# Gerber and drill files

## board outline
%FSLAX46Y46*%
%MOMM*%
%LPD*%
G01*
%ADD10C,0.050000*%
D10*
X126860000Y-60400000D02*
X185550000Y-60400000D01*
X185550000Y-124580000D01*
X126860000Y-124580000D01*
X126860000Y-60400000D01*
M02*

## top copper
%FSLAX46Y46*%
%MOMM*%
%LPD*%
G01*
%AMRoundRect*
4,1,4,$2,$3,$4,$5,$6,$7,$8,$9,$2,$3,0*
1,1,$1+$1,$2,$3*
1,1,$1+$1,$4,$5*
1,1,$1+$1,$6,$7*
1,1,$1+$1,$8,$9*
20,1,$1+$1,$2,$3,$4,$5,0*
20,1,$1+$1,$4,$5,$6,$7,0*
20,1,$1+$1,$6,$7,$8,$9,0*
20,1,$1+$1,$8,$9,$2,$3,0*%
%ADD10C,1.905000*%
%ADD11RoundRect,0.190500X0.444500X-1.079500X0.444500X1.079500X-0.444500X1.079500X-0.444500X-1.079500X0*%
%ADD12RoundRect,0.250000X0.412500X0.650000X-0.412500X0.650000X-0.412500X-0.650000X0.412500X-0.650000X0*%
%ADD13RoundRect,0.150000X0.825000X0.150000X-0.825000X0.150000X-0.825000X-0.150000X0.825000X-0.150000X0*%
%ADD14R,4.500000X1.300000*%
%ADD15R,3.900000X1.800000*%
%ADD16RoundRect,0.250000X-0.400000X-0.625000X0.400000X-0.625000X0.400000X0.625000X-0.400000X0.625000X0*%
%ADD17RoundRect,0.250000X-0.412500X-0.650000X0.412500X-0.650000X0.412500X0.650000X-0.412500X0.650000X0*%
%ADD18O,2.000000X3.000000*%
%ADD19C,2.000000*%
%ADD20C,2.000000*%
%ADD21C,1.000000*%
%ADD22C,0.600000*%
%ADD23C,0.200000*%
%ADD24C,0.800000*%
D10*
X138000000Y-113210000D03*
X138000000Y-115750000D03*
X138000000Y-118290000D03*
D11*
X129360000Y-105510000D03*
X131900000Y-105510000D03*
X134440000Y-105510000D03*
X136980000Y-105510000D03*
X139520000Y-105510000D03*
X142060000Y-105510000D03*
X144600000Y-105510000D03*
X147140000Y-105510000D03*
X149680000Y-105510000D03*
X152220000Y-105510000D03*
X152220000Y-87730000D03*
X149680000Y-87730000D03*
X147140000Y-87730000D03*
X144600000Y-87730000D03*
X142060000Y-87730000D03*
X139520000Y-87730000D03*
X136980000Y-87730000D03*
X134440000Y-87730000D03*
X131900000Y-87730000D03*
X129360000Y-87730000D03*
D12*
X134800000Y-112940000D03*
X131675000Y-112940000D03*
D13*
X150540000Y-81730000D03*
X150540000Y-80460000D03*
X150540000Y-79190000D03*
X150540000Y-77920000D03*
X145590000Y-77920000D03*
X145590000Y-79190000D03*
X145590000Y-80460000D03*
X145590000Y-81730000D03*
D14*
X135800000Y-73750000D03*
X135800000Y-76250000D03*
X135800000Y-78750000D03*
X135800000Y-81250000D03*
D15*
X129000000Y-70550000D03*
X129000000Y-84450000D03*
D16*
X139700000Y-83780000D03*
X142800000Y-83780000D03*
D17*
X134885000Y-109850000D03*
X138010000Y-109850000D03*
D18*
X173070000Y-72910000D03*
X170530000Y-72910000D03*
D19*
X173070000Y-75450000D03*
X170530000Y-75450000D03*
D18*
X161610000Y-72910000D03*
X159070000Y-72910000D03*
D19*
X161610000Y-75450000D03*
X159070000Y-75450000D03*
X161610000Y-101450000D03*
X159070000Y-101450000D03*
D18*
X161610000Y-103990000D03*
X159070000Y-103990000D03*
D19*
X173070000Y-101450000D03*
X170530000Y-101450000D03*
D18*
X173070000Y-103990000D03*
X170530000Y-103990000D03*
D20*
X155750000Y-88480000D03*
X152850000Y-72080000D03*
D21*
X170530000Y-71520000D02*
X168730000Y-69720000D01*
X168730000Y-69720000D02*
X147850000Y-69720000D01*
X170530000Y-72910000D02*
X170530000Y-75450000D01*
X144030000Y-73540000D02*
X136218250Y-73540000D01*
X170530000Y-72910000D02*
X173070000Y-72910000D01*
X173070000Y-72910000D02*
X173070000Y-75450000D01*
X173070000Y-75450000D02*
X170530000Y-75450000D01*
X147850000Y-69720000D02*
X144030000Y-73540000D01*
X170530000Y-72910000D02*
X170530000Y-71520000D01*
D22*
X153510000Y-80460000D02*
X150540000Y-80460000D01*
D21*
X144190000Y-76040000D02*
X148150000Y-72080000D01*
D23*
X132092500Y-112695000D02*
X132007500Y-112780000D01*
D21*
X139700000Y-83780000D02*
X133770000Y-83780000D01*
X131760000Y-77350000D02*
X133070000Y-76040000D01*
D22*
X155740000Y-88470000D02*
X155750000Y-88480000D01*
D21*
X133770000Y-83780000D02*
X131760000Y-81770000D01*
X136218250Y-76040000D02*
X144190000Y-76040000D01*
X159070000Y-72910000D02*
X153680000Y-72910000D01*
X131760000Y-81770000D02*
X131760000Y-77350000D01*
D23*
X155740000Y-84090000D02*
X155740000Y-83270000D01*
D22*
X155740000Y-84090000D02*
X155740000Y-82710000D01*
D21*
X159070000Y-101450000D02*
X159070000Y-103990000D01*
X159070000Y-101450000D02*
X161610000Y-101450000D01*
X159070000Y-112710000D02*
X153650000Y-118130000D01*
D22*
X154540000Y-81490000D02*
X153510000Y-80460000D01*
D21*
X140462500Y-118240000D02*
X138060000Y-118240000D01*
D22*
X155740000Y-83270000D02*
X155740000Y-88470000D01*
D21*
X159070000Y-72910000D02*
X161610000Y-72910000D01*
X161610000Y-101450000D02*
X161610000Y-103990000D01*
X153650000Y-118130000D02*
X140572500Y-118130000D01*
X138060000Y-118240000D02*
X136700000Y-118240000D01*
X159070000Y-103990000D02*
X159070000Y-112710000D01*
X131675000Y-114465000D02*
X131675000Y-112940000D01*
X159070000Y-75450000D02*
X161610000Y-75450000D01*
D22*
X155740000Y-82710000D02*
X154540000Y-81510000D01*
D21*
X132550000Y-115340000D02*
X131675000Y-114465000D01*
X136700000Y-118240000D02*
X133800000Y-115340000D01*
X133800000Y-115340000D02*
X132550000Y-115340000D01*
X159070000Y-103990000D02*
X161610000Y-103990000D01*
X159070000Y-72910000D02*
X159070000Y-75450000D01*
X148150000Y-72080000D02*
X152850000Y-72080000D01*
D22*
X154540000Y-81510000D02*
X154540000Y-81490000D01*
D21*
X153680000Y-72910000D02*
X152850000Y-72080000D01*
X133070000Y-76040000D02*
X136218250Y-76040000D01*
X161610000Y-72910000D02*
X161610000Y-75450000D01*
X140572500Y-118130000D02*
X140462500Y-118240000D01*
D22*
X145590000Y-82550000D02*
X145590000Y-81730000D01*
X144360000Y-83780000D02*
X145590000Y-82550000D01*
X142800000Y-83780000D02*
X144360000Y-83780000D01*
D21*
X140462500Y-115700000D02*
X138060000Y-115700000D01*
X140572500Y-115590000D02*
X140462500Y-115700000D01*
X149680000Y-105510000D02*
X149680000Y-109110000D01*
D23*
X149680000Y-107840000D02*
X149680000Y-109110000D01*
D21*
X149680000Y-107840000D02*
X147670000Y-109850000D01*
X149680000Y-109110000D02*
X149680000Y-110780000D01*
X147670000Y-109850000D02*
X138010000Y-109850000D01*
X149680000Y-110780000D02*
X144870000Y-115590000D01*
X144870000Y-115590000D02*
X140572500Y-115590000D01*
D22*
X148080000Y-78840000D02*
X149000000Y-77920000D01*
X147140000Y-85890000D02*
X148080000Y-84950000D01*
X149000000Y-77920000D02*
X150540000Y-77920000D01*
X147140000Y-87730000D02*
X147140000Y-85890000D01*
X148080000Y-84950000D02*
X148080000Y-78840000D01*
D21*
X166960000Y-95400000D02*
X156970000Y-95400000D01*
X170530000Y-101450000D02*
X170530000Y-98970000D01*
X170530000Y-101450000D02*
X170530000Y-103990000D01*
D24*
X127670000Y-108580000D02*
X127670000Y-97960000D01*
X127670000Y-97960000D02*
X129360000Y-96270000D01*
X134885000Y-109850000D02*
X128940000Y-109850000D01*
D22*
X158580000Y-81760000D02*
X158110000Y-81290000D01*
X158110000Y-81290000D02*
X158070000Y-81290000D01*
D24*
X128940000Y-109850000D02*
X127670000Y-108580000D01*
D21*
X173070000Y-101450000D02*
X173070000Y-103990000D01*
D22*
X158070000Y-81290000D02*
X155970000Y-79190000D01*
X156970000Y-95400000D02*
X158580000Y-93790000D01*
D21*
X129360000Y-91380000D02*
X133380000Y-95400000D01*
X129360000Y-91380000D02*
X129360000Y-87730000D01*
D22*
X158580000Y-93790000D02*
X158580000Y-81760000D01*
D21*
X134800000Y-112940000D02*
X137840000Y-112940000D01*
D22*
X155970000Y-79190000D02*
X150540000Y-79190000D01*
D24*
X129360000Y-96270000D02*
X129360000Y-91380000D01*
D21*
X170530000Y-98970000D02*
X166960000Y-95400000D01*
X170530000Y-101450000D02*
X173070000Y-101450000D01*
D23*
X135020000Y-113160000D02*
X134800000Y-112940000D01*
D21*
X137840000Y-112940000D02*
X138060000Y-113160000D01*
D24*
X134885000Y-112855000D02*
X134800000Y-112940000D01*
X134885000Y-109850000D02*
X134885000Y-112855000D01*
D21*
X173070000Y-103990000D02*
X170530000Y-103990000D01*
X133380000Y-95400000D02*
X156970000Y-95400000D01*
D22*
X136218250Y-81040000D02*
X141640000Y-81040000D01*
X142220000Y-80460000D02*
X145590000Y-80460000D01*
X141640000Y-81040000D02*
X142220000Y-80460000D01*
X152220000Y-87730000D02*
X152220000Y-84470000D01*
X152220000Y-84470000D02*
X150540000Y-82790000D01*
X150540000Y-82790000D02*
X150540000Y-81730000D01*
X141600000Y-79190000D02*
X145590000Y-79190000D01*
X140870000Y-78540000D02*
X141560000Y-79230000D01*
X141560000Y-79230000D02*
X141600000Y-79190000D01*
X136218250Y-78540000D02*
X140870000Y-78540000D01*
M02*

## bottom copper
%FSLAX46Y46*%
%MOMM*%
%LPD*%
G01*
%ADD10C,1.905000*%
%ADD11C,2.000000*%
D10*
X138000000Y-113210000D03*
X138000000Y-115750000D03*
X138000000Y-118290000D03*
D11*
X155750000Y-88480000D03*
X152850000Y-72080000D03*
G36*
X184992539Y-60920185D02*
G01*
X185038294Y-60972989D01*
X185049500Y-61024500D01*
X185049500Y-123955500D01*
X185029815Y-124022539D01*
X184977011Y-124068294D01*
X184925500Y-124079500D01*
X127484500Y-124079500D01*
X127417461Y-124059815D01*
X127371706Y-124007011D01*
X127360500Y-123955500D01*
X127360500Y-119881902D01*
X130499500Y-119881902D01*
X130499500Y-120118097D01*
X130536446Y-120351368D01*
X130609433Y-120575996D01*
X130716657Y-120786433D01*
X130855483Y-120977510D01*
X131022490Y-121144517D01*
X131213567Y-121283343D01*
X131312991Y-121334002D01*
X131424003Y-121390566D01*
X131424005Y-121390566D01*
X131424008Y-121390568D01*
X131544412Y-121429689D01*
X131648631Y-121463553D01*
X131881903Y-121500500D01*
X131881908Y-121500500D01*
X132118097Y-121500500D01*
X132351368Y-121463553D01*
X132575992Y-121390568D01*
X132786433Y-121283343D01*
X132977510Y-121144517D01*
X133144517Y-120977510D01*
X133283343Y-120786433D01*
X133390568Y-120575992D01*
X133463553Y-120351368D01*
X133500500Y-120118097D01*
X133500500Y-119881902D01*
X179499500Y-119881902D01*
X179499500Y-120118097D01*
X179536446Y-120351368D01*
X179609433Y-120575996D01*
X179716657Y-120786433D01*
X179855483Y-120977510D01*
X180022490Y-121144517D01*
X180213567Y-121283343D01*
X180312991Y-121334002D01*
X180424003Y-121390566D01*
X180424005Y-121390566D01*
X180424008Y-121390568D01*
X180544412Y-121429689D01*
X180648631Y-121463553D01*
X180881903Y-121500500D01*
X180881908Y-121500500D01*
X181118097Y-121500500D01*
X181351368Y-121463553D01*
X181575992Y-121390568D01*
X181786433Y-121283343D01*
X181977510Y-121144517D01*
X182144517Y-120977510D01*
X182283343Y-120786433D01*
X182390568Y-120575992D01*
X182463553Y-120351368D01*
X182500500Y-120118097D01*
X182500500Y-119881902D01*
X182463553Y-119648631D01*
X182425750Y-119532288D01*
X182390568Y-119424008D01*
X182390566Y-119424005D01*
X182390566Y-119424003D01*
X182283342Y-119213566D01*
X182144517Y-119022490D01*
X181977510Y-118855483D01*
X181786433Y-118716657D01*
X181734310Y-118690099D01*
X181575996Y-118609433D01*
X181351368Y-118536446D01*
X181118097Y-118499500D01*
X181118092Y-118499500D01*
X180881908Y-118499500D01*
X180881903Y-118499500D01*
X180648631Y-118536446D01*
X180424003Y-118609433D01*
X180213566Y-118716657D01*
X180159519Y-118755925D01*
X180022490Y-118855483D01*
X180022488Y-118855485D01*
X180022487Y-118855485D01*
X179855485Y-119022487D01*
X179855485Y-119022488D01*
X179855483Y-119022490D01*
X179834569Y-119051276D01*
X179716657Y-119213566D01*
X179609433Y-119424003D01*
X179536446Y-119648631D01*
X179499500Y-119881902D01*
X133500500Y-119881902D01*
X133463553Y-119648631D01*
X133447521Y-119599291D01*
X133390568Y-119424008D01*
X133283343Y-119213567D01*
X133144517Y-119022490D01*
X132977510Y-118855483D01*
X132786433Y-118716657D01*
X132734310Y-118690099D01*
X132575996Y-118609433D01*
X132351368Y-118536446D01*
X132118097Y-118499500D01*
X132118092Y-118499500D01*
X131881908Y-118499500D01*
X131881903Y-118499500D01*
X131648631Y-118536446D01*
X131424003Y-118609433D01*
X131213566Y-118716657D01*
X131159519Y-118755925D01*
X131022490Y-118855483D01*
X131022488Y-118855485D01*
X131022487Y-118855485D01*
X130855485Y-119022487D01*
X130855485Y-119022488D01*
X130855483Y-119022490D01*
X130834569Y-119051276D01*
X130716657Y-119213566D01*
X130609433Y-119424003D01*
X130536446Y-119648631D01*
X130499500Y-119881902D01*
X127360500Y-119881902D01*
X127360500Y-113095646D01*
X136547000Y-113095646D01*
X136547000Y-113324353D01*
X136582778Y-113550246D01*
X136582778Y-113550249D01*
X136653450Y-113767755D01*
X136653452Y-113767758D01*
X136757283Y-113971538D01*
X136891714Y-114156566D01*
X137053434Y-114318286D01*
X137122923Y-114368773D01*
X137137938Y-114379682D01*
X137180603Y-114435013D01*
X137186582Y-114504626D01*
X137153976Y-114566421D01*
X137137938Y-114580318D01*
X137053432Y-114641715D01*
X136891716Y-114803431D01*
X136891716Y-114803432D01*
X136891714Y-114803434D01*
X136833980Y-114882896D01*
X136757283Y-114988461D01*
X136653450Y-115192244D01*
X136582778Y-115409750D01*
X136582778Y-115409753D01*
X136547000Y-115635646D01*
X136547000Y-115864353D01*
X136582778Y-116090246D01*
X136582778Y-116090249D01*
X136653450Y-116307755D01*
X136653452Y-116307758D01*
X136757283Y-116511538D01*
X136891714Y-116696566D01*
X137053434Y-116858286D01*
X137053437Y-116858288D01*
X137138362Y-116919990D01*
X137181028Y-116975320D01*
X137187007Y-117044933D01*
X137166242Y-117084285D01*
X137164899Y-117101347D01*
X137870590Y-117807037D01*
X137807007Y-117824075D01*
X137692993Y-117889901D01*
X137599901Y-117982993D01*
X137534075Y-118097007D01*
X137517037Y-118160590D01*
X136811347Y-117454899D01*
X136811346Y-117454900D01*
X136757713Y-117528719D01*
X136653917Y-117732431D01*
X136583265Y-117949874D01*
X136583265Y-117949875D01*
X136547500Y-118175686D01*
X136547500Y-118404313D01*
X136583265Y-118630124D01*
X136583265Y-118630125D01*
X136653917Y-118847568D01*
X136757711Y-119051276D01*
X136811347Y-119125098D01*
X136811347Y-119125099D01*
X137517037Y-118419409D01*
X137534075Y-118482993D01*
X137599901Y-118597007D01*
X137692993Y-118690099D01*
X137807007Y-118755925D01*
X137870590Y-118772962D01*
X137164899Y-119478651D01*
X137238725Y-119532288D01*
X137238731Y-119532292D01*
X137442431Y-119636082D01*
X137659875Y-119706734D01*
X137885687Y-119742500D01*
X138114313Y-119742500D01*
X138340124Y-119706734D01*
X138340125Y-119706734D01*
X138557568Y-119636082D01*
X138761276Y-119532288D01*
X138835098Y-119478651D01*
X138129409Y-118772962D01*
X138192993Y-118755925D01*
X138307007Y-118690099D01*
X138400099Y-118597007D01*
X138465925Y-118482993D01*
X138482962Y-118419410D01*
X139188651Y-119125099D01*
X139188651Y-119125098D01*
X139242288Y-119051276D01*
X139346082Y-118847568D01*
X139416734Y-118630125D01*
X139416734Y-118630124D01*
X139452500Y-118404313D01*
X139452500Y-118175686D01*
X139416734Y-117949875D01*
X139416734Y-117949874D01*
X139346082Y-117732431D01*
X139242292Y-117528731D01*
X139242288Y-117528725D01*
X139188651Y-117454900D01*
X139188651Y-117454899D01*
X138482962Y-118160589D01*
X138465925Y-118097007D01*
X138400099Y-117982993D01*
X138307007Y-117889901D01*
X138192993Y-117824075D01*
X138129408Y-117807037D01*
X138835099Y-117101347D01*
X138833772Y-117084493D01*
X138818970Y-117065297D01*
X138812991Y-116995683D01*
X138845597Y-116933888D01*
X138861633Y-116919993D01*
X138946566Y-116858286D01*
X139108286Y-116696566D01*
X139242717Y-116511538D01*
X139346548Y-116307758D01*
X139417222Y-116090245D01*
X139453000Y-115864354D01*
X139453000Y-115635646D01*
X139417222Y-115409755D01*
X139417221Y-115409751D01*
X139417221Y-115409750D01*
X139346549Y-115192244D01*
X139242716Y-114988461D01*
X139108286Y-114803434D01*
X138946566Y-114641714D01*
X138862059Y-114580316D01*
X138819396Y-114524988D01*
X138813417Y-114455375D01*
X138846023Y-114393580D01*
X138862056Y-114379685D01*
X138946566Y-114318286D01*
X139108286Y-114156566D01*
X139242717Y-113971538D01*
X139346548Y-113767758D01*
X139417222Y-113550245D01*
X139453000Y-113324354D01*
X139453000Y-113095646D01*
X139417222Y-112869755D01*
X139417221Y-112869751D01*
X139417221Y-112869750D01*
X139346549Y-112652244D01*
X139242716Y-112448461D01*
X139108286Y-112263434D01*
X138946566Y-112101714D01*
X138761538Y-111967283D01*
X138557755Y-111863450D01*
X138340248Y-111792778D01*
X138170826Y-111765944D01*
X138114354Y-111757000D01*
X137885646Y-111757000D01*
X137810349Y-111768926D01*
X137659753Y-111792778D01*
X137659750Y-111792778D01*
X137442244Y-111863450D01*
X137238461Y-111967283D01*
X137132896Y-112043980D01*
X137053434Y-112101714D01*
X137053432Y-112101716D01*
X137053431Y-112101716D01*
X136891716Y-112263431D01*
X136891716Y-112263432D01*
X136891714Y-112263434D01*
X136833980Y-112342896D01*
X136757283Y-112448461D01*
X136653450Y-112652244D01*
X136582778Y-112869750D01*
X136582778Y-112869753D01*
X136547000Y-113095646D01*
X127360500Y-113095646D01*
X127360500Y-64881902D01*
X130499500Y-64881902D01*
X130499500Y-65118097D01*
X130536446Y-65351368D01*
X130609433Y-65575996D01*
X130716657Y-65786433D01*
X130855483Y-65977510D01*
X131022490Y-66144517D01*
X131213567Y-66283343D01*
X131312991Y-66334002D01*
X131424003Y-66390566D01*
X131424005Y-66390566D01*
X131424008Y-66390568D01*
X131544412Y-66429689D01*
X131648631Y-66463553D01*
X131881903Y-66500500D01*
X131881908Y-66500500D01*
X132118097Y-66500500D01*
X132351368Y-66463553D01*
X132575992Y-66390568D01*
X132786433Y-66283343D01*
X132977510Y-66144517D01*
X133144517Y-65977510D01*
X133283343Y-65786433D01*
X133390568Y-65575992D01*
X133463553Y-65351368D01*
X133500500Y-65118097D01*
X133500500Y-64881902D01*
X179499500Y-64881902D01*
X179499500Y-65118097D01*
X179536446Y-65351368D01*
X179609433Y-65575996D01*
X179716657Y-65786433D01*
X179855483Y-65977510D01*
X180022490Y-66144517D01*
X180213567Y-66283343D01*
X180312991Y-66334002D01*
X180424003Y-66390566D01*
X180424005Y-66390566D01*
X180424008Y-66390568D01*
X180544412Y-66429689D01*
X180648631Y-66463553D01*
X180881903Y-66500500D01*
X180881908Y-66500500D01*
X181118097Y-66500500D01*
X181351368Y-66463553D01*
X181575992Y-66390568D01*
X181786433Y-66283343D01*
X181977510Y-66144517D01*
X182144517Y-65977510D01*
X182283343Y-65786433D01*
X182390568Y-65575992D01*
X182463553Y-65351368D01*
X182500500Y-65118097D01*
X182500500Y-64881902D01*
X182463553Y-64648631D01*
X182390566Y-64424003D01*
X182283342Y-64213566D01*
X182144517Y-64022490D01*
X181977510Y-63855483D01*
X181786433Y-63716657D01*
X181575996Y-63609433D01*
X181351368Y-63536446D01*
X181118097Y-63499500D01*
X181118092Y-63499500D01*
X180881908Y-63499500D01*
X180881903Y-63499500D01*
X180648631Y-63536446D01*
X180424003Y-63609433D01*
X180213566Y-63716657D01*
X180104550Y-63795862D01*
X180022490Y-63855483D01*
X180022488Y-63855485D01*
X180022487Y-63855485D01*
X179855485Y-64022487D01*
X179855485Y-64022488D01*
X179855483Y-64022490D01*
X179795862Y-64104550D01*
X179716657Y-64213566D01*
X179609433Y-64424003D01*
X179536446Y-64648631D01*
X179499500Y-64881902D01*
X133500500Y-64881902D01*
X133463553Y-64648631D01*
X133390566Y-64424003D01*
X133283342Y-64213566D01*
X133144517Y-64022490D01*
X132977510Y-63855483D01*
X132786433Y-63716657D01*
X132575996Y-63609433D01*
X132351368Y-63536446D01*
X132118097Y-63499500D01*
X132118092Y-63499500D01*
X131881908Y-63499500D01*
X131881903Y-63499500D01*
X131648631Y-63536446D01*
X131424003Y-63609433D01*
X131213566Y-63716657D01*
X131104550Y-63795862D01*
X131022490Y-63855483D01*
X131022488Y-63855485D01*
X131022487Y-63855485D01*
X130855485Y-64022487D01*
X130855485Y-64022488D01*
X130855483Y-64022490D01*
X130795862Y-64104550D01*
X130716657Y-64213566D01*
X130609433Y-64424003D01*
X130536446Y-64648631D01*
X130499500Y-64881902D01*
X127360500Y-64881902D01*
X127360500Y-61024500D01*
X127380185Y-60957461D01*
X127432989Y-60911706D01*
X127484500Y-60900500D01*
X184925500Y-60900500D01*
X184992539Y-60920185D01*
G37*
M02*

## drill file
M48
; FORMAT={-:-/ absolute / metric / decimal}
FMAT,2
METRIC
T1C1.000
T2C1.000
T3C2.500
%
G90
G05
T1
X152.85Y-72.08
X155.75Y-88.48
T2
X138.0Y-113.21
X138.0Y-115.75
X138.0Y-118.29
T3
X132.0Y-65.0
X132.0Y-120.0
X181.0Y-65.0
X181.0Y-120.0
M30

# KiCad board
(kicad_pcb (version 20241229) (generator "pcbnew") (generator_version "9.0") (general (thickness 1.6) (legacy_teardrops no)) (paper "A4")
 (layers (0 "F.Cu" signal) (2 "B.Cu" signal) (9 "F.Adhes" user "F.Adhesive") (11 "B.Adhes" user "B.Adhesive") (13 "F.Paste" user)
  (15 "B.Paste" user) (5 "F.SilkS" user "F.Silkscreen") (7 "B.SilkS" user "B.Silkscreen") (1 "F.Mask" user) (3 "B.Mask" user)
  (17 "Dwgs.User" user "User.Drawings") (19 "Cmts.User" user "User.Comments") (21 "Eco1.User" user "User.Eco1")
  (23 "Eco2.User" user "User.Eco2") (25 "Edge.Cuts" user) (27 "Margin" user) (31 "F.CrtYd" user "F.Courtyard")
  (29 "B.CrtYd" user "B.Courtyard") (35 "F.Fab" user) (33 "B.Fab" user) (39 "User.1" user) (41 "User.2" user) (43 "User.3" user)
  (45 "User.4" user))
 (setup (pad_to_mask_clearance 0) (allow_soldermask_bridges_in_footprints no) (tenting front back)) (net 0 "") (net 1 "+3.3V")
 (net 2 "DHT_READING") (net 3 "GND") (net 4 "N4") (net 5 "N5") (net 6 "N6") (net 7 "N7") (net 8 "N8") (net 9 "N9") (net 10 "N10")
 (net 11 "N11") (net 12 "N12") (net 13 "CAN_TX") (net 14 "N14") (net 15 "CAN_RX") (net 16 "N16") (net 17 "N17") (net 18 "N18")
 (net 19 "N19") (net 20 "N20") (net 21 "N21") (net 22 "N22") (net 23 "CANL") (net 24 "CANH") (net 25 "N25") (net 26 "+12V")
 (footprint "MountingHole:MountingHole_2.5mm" (layer "F.Cu") (at 181 65)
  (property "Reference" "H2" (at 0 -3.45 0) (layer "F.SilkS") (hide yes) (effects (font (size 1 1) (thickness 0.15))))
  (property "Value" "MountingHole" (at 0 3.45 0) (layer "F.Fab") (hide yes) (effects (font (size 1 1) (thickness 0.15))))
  (pad "" np_thru_hole circle (at 0 0) (size 2.5 2.5) (drill 2.5) (layers "*.Cu" "*.Mask")))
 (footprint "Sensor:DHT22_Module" (layer "F.Cu") (at 143.08 110.67 180)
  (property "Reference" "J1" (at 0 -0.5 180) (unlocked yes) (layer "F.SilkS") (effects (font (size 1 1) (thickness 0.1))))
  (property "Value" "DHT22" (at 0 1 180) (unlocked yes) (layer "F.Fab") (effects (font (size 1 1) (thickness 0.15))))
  (pad "1" thru_hole circle (at 5.08 -2.54 180) (size 1.905 1.905) (drill 1) (layers "*.Cu" "*.Mask") (remove_unused_layers no)
   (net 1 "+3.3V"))
  (pad "2" thru_hole circle (at 5.08 -5.08 180) (size 1.905 1.905) (drill 1) (layers "*.Cu" "*.Mask") (remove_unused_layers no)
   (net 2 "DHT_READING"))
  (pad "3" thru_hole circle (at 5.08 -7.62 180) (size 1.905 1.905) (drill 1) (layers "*.Cu" "*.Mask") (remove_unused_layers no)
   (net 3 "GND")))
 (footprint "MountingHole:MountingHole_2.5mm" (layer "F.Cu") (at 132 65)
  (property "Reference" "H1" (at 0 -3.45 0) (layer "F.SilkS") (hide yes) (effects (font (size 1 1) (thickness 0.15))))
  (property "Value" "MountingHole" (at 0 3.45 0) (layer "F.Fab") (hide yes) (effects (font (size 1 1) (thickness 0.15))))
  (pad "" np_thru_hole circle (at 0 0) (size 2.5 2.5) (drill 2.5) (layers "*.Cu" "*.Mask")))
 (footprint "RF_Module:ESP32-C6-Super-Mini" (layer "F.Cu") (at 157.338 110.165 90)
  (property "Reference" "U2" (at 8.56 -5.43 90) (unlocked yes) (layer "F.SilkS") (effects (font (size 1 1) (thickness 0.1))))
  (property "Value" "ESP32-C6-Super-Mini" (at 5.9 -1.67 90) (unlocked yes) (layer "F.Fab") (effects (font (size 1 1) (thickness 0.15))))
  (pad "1" smd roundrect (at 4.655 -27.978 90) (size 2.54 1.27) (layers "F.Cu" "F.Mask" "F.Paste") (roundrect_rratio 0.15) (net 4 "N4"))
  (pad "2" smd roundrect (at 4.655 -25.438 90) (size 2.54 1.27) (layers "F.Cu" "F.Mask" "F.Paste") (roundrect_rratio 0.15) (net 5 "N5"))
  (pad "3" smd roundrect (at 4.655 -22.898 90) (size 2.54 1.27) (layers "F.Cu" "F.Mask" "F.Paste") (roundrect_rratio 0.15) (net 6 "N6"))
  (pad "4" smd roundrect (at 4.655 -20.358 90) (size 2.54 1.27) (layers "F.Cu" "F.Mask" "F.Paste") (roundrect_rratio 0.15) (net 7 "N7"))
  (pad "5" smd roundrect (at 4.655 -17.818 90) (size 2.54 1.27) (layers "F.Cu" "F.Mask" "F.Paste") (roundrect_rratio 0.15) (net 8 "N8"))
  (pad "6" smd roundrect (at 4.655 -15.278 90) (size 2.54 1.27) (layers "F.Cu" "F.Mask" "F.Paste") (roundrect_rratio 0.15) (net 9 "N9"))
  (pad "7" smd roundrect (at 4.655 -12.738 90) (size 2.54 1.27) (layers "F.Cu" "F.Mask" "F.Paste") (roundrect_rratio 0.15) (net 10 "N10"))
  (pad "8" smd roundrect (at 4.655 -10.198 90) (size 2.54 1.27) (layers "F.Cu" "F.Mask" "F.Paste") (roundrect_rratio 0.15) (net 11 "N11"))
  (pad "9" smd roundrect (at 4.655 -7.658 90) (size 2.54 1.27) (layers "F.Cu" "F.Mask" "F.Paste") (roundrect_rratio 0.15)
   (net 2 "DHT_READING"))
  (pad "10" smd roundrect (at 4.655 -5.118 90) (size 2.54 1.27) (layers "F.Cu" "F.Mask" "F.Paste") (roundrect_rratio 0.15) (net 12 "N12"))
  (pad "11" smd roundrect (at 22.435 -5.118 90) (size 2.54 1.27) (layers "F.Cu" "F.Mask" "F.Paste") (roundrect_rratio 0.15)
   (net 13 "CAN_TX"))
  (pad "12" smd roundrect (at 22.435 -7.658 90) (size 2.54 1.27) (layers "F.Cu" "F.Mask" "F.Paste") (roundrect_rratio 0.15) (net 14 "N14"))
  (pad "13" smd roundrect (at 22.435 -10.198 90) (size 2.54 1.27) (layers "F.Cu" "F.Mask" "F.Paste") (roundrect_rratio 0.15)
   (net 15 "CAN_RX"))
  (pad "14" smd roundrect (at 22.435 -12.738 90) (size 2.54 1.27) (layers "F.Cu" "F.Mask" "F.Paste") (roundrect_rratio 0.15) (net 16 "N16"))
  (pad "15" smd roundrect (at 22.435 -15.278 90) (size 2.54 1.27) (layers "F.Cu" "F.Mask" "F.Paste") (roundrect_rratio 0.15) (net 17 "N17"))
  (pad "16" smd roundrect (at 22.435 -17.818 90) (size 2.54 1.27) (layers "F.Cu" "F.Mask" "F.Paste") (roundrect_rratio 0.15) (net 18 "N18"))
  (pad "17" smd roundrect (at 22.435 -20.358 90) (size 2.54 1.27) (layers "F.Cu" "F.Mask" "F.Paste") (roundrect_rratio 0.15) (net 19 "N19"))
  (pad "18" smd roundrect (at 22.435 -22.898 90) (size 2.54 1.27) (layers "F.Cu" "F.Mask" "F.Paste") (roundrect_rratio 0.15) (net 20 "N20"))
  (pad "19" smd roundrect (at 22.435 -25.438 90) (size 2.54 1.27) (layers "F.Cu" "F.Mask" "F.Paste") (roundrect_rratio 0.15) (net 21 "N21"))
  (pad "20" smd roundrect (at 22.435 -27.978 90) (size 2.54 1.27) (layers "F.Cu" "F.Mask" "F.Paste") (roundrect_rratio 0.15) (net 1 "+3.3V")))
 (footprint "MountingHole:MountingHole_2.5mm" (layer "F.Cu") (at 132 120)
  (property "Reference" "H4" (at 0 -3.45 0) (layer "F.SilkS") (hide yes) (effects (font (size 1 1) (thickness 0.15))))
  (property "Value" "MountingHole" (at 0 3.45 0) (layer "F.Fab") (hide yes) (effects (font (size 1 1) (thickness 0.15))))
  (pad "" np_thru_hole circle (at 0 0) (size 2.5 2.5) (drill 2.5) (layers "*.Cu" "*.Mask")))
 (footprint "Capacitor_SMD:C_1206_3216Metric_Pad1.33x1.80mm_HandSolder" (layer "F.Cu") (at 133.2375 112.94 180)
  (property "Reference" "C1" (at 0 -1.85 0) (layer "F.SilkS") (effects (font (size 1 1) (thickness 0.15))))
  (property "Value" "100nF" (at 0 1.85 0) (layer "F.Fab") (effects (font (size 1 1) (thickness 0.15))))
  (pad "1" smd roundrect (at -1.5625 0 180) (size 1.325 1.8) (layers "F.Cu" "F.Mask" "F.Paste") (roundrect_rratio 0.188679) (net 1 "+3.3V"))
  (pad "2" smd roundrect (at 1.5625 0 180) (size 1.325 1.8) (layers "F.Cu" "F.Mask" "F.Paste") (roundrect_rratio 0.188679) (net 3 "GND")))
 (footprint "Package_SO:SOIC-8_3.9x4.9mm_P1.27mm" (layer "F.Cu") (at 148.065 79.825 180)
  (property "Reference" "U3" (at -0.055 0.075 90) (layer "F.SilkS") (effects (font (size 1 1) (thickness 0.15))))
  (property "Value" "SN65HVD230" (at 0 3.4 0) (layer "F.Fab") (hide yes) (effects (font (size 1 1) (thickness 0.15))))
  (pad "1" smd roundrect (at -2.475 -1.905 180) (size 1.95 0.6) (layers "F.Cu" "F.Mask" "F.Paste") (roundrect_rratio 0.25) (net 13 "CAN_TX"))
  (pad "2" smd roundrect (at -2.475 -0.635 180) (size 1.95 0.6) (layers "F.Cu" "F.Mask" "F.Paste") (roundrect_rratio 0.25) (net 3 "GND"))
  (pad "3" smd roundrect (at -2.475 0.635 180) (size 1.95 0.6) (layers "F.Cu" "F.Mask" "F.Paste") (roundrect_rratio 0.25) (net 1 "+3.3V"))
  (pad "4" smd roundrect (at -2.475 1.905 180) (size 1.95 0.6) (layers "F.Cu" "F.Mask" "F.Paste") (roundrect_rratio 0.25) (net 15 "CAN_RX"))
  (pad "5" smd roundrect (at 2.475 1.905 180) (size 1.95 0.6) (layers "F.Cu" "F.Mask" "F.Paste") (roundrect_rratio 0.25) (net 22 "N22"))
  (pad "6" smd roundrect (at 2.475 0.635 180) (size 1.95 0.6) (layers "F.Cu" "F.Mask" "F.Paste") (roundrect_rratio 0.25) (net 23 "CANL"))
  (pad "7" smd roundrect (at 2.475 -0.635 180) (size 1.95 0.6) (layers "F.Cu" "F.Mask" "F.Paste") (roundrect_rratio 0.25) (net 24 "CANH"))
  (pad "8" smd roundrect (at 2.475 -1.905 180) (size 1.95 0.6) (layers "F.Cu" "F.Mask" "F.Paste") (roundrect_rratio 0.25) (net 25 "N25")))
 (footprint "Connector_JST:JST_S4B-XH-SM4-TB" (layer "F.Cu") (at 129 77.5 -90)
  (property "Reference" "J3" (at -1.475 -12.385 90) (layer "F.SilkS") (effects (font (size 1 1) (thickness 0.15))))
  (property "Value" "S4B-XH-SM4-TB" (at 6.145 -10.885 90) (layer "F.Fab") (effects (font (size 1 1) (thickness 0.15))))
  (pad "1" smd rect (at -3.75 -6.8 270) (size 1.3 4.5) (layers "F.Cu" "F.Mask" "F.Paste") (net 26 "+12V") (solder_mask_margin 0.102))
  (pad "2" smd rect (at -1.25 -6.8 270) (size 1.3 4.5) (layers "F.Cu" "F.Mask" "F.Paste") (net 3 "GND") (solder_mask_margin 0.102))
  (pad "3" smd rect (at 1.25 -6.8 270) (size 1.3 4.5) (layers "F.Cu" "F.Mask" "F.Paste") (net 23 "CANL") (solder_mask_margin 0.102))
  (pad "4" smd rect (at 3.75 -6.8 270) (size 1.3 4.5) (layers "F.Cu" "F.Mask" "F.Paste") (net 24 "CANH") (solder_mask_margin 0.102))
  (pad "SH1" smd rect (at -6.95 0 270) (size 1.8 3.9) (layers "F.Cu" "F.Mask" "F.Paste") (solder_mask_margin 0.102))
  (pad "SH2" smd rect (at 6.95 0 270) (size 1.8 3.9) (layers "F.Cu" "F.Mask" "F.Paste") (solder_mask_margin 0.102)))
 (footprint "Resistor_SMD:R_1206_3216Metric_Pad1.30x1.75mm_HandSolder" (layer "F.Cu") (at 141.25 83.78)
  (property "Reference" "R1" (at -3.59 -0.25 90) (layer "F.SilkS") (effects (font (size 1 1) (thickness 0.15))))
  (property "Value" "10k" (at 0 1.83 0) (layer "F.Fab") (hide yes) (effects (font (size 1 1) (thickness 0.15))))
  (pad "1" smd roundrect (at -1.55 0) (size 1.3 1.75) (layers "F.Cu" "F.Mask" "F.Paste") (roundrect_rratio 0.192308) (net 3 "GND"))
  (pad "2" smd roundrect (at 1.55 0) (size 1.3 1.75) (layers "F.Cu" "F.Mask" "F.Paste") (roundrect_rratio 0.192308) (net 25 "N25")))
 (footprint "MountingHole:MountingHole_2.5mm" (layer "F.Cu") (at 181 120)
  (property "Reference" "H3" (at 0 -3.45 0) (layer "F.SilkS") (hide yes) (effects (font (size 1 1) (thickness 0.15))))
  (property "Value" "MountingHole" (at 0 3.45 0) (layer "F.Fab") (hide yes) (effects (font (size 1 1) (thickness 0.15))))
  (pad "" np_thru_hole circle (at 0 0) (size 2.5 2.5) (drill 2.5) (layers "*.Cu" "*.Mask")))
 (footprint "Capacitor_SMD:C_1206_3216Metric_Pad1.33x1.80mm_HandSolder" (layer "F.Cu") (at 136.4475 109.85)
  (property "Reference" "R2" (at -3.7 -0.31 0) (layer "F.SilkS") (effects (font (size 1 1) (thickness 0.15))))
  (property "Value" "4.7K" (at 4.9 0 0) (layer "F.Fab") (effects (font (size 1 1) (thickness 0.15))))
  (pad "1" smd roundrect (at -1.5625 0) (size 1.325 1.8) (layers "F.Cu" "F.Mask" "F.Paste") (roundrect_rratio 0.188679) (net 1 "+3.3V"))
  (pad "2" smd roundrect (at 1.5625 0) (size 1.325 1.8) (layers "F.Cu" "F.Mask" "F.Paste") (roundrect_rratio 0.188679) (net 2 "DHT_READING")))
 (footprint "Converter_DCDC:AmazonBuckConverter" (layer "F.Cu") (at 153.99 75.45 -90)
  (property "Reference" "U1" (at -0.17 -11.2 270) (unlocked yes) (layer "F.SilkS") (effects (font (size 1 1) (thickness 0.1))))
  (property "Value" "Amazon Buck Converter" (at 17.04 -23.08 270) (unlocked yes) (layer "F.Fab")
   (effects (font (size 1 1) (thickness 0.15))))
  (pad "1" smd oval (at -2.54 -19.08) (size 2 3) (layers "F.Cu" "F.Mask" "F.Paste") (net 26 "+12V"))
  (pad "1" smd oval (at -2.54 -16.54) (size 2 3) (layers "F.Cu" "F.Mask" "F.Paste") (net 26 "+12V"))
  (pad "1" smd circle (at 0 -19.08) (size 2 2) (layers "F.Cu" "F.Mask" "F.Paste") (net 26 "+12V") (thermal_bridge_angle 90))
  (pad "1" smd circle (at 0 -16.54) (size 2 2) (layers "F.Cu" "F.Mask" "F.Paste") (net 26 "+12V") (thermal_bridge_angle 90))
  (pad "2" smd oval (at -2.54 -7.62) (size 2 3) (layers "F.Cu" "F.Mask" "F.Paste") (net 3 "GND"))
  (pad "2" smd oval (at -2.54 -5.08) (size 2 3) (layers "F.Cu" "F.Mask" "F.Paste") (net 3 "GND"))
  (pad "2" smd circle (at 0 -7.62) (size 2 2) (layers "F.Cu" "F.Mask" "F.Paste") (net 3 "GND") (thermal_bridge_angle 90))
  (pad "2" smd circle (at 0 -5.08) (size 2 2) (layers "F.Cu" "F.Mask" "F.Paste") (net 3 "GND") (thermal_bridge_angle 90))
  (pad "3" smd circle (at 26 -7.62) (size 2 2) (layers "F.Cu" "F.Mask" "F.Paste") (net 3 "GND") (thermal_bridge_angle 90))
  (pad "3" smd circle (at 26 -5.08) (size 2 2) (layers "F.Cu" "F.Mask" "F.Paste") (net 3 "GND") (thermal_bridge_angle 90))
  (pad "3" smd oval (at 28.54 -7.62) (size 2 3) (layers "F.Cu" "F.Mask" "F.Paste") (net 3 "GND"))
  (pad "3" smd oval (at 28.54 -5.08) (size 2 3) (layers "F.Cu" "F.Mask" "F.Paste") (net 3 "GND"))
  (pad "4" smd circle (at 26 -19.08) (size 2 2) (layers "F.Cu" "F.Mask" "F.Paste") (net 1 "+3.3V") (thermal_bridge_angle 90))
  (pad "4" smd circle (at 26 -16.54) (size 2 2) (layers "F.Cu" "F.Mask" "F.Paste") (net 1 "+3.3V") (thermal_bridge_angle 90))
  (pad "4" smd oval (at 28.54 -19.08) (size 2 3) (layers "F.Cu" "F.Mask" "F.Paste") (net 1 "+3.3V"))
  (pad "4" smd oval (at 28.54 -16.54) (size 2 3) (layers "F.Cu" "F.Mask" "F.Paste") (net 1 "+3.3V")))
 (gr_rect (start 126.86 60.4) (end 185.55 124.58) (stroke (width 0.05) (type default)) (fill no) (layer "Edge.Cuts"))
 (segment (start 170.53 71.52) (end 168.73 69.72) (width 1) (layer "F.Cu") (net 26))
 (segment (start 168.73 69.72) (end 147.85 69.72) (width 1) (layer "F.Cu") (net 26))
 (segment (start 170.53 72.91) (end 170.53 75.45) (width 1) (layer "F.Cu") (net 26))
 (segment (start 144.03 73.54) (end 136.21825 73.54) (width 1) (layer "F.Cu") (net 26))
 (segment (start 170.53 72.91) (end 173.07 72.91) (width 1) (layer "F.Cu") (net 26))
 (segment (start 173.07 72.91) (end 173.07 75.45) (width 1) (layer "F.Cu") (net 26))
 (segment (start 173.07 75.45) (end 170.53 75.45) (width 1) (layer "F.Cu") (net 26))
 (segment (start 147.85 69.72) (end 144.03 73.54) (width 1) (layer "F.Cu") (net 26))
 (segment (start 170.53 72.91) (end 170.53 71.52) (width 1) (layer "F.Cu") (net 26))
 (segment (start 153.51 80.46) (end 150.54 80.46) (width 0.6) (layer "F.Cu") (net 3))
 (segment (start 144.19 76.04) (end 148.15 72.08) (width 1) (layer "F.Cu") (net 3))
 (segment (start 132.0925 112.695) (end 132.0075 112.78) (width 0.2) (layer "F.Cu") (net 3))
 (segment (start 139.7 83.78) (end 133.77 83.78) (width 1) (layer "F.Cu") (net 3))
 (segment (start 131.76 77.35) (end 133.07 76.04) (width 1) (layer "F.Cu") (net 3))
 (segment (start 155.74 88.47) (end 155.75 88.48) (width 0.6) (layer "F.Cu") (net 3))
 (segment (start 133.77 83.78) (end 131.76 81.77) (width 1) (layer "F.Cu") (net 3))
 (segment (start 136.21825 76.04) (end 144.19 76.04) (width 1) (layer "F.Cu") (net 3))
 (segment (start 159.07 72.91) (end 153.68 72.91) (width 1) (layer "F.Cu") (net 3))
 (segment (start 131.76 81.77) (end 131.76 77.35) (width 1) (layer "F.Cu") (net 3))
 (segment (start 155.74 84.09) (end 155.74 83.27) (width 0.2) (layer "F.Cu") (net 3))
 (segment (start 155.74 84.09) (end 155.74 82.71) (width 0.6) (layer "F.Cu") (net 3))
 (segment (start 159.07 101.45) (end 159.07 103.99) (width 1) (layer "F.Cu") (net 3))
 (segment (start 159.07 101.45) (end 161.61 101.45) (width 1) (layer "F.Cu") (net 3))
 (segment (start 159.07 112.71) (end 153.65 118.13) (width 1) (layer "F.Cu") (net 3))
 (segment (start 154.54 81.49) (end 153.51 80.46) (width 0.6) (layer "F.Cu") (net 3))
 (segment (start 140.4625 118.24) (end 138.06 118.24) (width 1) (layer "F.Cu") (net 3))
 (segment (start 155.74 83.27) (end 155.74 88.47) (width 0.6) (layer "F.Cu") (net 3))
 (segment (start 159.07 72.91) (end 161.61 72.91) (width 1) (layer "F.Cu") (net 3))
 (segment (start 161.61 101.45) (end 161.61 103.99) (width 1) (layer "F.Cu") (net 3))
 (segment (start 153.65 118.13) (end 140.5725 118.13) (width 1) (layer "F.Cu") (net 3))
 (segment (start 138.06 118.24) (end 136.7 118.24) (width 1) (layer "F.Cu") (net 3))
 (segment (start 159.07 103.99) (end 159.07 112.71) (width 1) (layer "F.Cu") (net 3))
 (segment (start 131.675 114.465) (end 131.675 112.94) (width 1) (layer "F.Cu") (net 3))
 (segment (start 159.07 75.45) (end 161.61 75.45) (width 1) (layer "F.Cu") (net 3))
 (segment (start 155.74 82.71) (end 154.54 81.51) (width 0.6) (layer "F.Cu") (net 3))
 (segment (start 132.55 115.34) (end 131.675 114.465) (width 1) (layer "F.Cu") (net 3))
 (segment (start 136.7 118.24) (end 133.8 115.34) (width 1) (layer "F.Cu") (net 3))
 (segment (start 133.8 115.34) (end 132.55 115.34) (width 1) (layer "F.Cu") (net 3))
 (segment (start 159.07 103.99) (end 161.61 103.99) (width 1) (layer "F.Cu") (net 3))
 (segment (start 159.07 72.91) (end 159.07 75.45) (width 1) (layer "F.Cu") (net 3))
 (segment (start 148.15 72.08) (end 152.85 72.08) (width 1) (layer "F.Cu") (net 3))
 (segment (start 154.54 81.51) (end 154.54 81.49) (width 0.6) (layer "F.Cu") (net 3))
 (segment (start 153.68 72.91) (end 152.85 72.08) (width 1) (layer "F.Cu") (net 3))
 (segment (start 133.07 76.04) (end 136.21825 76.04) (width 1) (layer "F.Cu") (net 3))
 (segment (start 161.61 72.91) (end 161.61 75.45) (width 1) (layer "F.Cu") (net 3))
 (segment (start 140.5725 118.13) (end 140.4625 118.24) (width 1) (layer "F.Cu") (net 3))
 (via (at 155.75 88.48) (size 2) (drill 1) (layers "F.Cu" "B.Cu") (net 3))
 (via (at 152.85 72.08) (size 2) (drill 1) (layers "F.Cu" "B.Cu") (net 3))
 (segment (start 145.59 82.55) (end 145.59 81.73) (width 0.6) (layer "F.Cu") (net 25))
 (segment (start 144.36 83.78) (end 145.59 82.55) (width 0.6) (layer "F.Cu") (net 25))
 (segment (start 142.8 83.78) (end 144.36 83.78) (width 0.6) (layer "F.Cu") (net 25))
 (segment (start 140.4625 115.7) (end 138.06 115.7) (width 1) (layer "F.Cu") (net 2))
 (segment (start 140.5725 115.59) (end 140.4625 115.7) (width 1) (layer "F.Cu") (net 2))
 (segment (start 149.68 105.51) (end 149.68 109.11) (width 1) (layer "F.Cu") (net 2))
 (segment (start 149.68 107.84) (end 149.68 109.11) (width 0.2) (layer "F.Cu") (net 2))
 (segment (start 149.68 107.84) (end 147.67 109.85) (width 1) (layer "F.Cu") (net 2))
 (segment (start 149.68 109.11) (end 149.68 110.78) (width 1) (layer "F.Cu") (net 2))
 (segment (start 147.67 109.85) (end 138.01 109.85) (width 1) (layer "F.Cu") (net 2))
 (segment (start 149.68 110.78) (end 144.87 115.59) (width 1) (layer "F.Cu") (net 2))
 (segment (start 144.87 115.59) (end 140.5725 115.59) (width 1) (layer "F.Cu") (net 2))
 (segment (start 148.08 78.84) (end 149 77.92) (width 0.6) (layer "F.Cu") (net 15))
 (segment (start 147.14 85.89) (end 148.08 84.95) (width 0.6) (layer "F.Cu") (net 15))
 (segment (start 149 77.92) (end 150.54 77.92) (width 0.6) (layer "F.Cu") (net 15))
 (segment (start 147.14 87.73) (end 147.14 85.89) (width 0.6) (layer "F.Cu") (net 15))
 (segment (start 148.08 84.95) (end 148.08 78.84) (width 0.6) (layer "F.Cu") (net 15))
 (segment (start 166.96 95.4) (end 156.97 95.4) (width 1) (layer "F.Cu") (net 1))
 (segment (start 170.53 101.45) (end 170.53 98.97) (width 1) (layer "F.Cu") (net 1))
 (segment (start 170.53 101.45) (end 170.53 103.99) (width 1) (layer "F.Cu") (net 1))
 (segment (start 127.67 108.58) (end 127.67 97.96) (width 0.8) (layer "F.Cu") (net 1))
 (segment (start 127.67 97.96) (end 129.36 96.27) (width 0.8) (layer "F.Cu") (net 1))
 (segment (start 134.885 109.85) (end 128.94 109.85) (width 0.8) (layer "F.Cu") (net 1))
 (segment (start 158.58 81.76) (end 158.11 81.29) (width 0.6) (layer "F.Cu") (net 1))
 (segment (start 158.11 81.29) (end 158.07 81.29) (width 0.6) (layer "F.Cu") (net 1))
 (segment (start 128.94 109.85) (end 127.67 108.58) (width 0.8) (layer "F.Cu") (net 1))
 (segment (start 173.07 101.45) (end 173.07 103.99) (width 1) (layer "F.Cu") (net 1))
 (segment (start 158.07 81.29) (end 155.97 79.19) (width 0.6) (layer "F.Cu") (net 1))
 (segment (start 156.97 95.4) (end 158.58 93.79) (width 0.6) (layer "F.Cu") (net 1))
 (segment (start 129.36 91.38) (end 133.38 95.4) (width 1) (layer "F.Cu") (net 1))
 (segment (start 129.36 91.38) (end 129.36 87.73) (width 1) (layer "F.Cu") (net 1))
 (segment (start 158.58 93.79) (end 158.58 81.76) (width 0.6) (layer "F.Cu") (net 1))
 (segment (start 134.8 112.94) (end 137.84 112.94) (width 1) (layer "F.Cu") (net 1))
 (segment (start 155.97 79.19) (end 150.54 79.19) (width 0.6) (layer "F.Cu") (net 1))
 (segment (start 129.36 96.27) (end 129.36 91.38) (width 0.8) (layer "F.Cu") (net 1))
 (segment (start 170.53 98.97) (end 166.96 95.4) (width 1) (layer "F.Cu") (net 1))
 (segment (start 170.53 101.45) (end 173.07 101.45) (width 1) (layer "F.Cu") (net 1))
 (segment (start 135.02 113.16) (end 134.8 112.94) (width 0.2) (layer "F.Cu") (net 1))
 (segment (start 137.84 112.94) (end 138.06 113.16) (width 1) (layer "F.Cu") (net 1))
 (segment (start 134.885 112.855) (end 134.8 112.94) (width 0.8) (layer "F.Cu") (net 1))
 (segment (start 134.885 109.85) (end 134.885 112.855) (width 0.8) (layer "F.Cu") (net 1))
 (segment (start 173.07 103.99) (end 170.53 103.99) (width 1) (layer "F.Cu") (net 1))
 (segment (start 133.38 95.4) (end 156.97 95.4) (width 1) (layer "F.Cu") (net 1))
 (segment (start 136.21825 81.04) (end 141.64 81.04) (width 0.6) (layer "F.Cu") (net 24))
 (segment (start 142.22 80.46) (end 145.59 80.46) (width 0.6) (layer "F.Cu") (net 24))
 (segment (start 141.64 81.04) (end 142.22 80.46) (width 0.6) (layer "F.Cu") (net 24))
 (segment (start 152.22 87.73) (end 152.22 84.47) (width 0.6) (layer "F.Cu") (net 13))
 (segment (start 152.22 84.47) (end 150.54 82.79) (width 0.6) (layer "F.Cu") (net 13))
 (segment (start 150.54 82.79) (end 150.54 81.73) (width 0.6) (layer "F.Cu") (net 13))
 (segment (start 141.6 79.19) (end 145.59 79.19) (width 0.6) (layer "F.Cu") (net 23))
 (segment (start 140.87 78.54) (end 141.56 79.23) (width 0.6) (layer "F.Cu") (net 23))
 (segment (start 141.56 79.23) (end 141.6 79.19) (width 0.6) (layer "F.Cu") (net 23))
 (segment (start 136.21825 78.54) (end 140.87 78.54) (width 0.6) (layer "F.Cu") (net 23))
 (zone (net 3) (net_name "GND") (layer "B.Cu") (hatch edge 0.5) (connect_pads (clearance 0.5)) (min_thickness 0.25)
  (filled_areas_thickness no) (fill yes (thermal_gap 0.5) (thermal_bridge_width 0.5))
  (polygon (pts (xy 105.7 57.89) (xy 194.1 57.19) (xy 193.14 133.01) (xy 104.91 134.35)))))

